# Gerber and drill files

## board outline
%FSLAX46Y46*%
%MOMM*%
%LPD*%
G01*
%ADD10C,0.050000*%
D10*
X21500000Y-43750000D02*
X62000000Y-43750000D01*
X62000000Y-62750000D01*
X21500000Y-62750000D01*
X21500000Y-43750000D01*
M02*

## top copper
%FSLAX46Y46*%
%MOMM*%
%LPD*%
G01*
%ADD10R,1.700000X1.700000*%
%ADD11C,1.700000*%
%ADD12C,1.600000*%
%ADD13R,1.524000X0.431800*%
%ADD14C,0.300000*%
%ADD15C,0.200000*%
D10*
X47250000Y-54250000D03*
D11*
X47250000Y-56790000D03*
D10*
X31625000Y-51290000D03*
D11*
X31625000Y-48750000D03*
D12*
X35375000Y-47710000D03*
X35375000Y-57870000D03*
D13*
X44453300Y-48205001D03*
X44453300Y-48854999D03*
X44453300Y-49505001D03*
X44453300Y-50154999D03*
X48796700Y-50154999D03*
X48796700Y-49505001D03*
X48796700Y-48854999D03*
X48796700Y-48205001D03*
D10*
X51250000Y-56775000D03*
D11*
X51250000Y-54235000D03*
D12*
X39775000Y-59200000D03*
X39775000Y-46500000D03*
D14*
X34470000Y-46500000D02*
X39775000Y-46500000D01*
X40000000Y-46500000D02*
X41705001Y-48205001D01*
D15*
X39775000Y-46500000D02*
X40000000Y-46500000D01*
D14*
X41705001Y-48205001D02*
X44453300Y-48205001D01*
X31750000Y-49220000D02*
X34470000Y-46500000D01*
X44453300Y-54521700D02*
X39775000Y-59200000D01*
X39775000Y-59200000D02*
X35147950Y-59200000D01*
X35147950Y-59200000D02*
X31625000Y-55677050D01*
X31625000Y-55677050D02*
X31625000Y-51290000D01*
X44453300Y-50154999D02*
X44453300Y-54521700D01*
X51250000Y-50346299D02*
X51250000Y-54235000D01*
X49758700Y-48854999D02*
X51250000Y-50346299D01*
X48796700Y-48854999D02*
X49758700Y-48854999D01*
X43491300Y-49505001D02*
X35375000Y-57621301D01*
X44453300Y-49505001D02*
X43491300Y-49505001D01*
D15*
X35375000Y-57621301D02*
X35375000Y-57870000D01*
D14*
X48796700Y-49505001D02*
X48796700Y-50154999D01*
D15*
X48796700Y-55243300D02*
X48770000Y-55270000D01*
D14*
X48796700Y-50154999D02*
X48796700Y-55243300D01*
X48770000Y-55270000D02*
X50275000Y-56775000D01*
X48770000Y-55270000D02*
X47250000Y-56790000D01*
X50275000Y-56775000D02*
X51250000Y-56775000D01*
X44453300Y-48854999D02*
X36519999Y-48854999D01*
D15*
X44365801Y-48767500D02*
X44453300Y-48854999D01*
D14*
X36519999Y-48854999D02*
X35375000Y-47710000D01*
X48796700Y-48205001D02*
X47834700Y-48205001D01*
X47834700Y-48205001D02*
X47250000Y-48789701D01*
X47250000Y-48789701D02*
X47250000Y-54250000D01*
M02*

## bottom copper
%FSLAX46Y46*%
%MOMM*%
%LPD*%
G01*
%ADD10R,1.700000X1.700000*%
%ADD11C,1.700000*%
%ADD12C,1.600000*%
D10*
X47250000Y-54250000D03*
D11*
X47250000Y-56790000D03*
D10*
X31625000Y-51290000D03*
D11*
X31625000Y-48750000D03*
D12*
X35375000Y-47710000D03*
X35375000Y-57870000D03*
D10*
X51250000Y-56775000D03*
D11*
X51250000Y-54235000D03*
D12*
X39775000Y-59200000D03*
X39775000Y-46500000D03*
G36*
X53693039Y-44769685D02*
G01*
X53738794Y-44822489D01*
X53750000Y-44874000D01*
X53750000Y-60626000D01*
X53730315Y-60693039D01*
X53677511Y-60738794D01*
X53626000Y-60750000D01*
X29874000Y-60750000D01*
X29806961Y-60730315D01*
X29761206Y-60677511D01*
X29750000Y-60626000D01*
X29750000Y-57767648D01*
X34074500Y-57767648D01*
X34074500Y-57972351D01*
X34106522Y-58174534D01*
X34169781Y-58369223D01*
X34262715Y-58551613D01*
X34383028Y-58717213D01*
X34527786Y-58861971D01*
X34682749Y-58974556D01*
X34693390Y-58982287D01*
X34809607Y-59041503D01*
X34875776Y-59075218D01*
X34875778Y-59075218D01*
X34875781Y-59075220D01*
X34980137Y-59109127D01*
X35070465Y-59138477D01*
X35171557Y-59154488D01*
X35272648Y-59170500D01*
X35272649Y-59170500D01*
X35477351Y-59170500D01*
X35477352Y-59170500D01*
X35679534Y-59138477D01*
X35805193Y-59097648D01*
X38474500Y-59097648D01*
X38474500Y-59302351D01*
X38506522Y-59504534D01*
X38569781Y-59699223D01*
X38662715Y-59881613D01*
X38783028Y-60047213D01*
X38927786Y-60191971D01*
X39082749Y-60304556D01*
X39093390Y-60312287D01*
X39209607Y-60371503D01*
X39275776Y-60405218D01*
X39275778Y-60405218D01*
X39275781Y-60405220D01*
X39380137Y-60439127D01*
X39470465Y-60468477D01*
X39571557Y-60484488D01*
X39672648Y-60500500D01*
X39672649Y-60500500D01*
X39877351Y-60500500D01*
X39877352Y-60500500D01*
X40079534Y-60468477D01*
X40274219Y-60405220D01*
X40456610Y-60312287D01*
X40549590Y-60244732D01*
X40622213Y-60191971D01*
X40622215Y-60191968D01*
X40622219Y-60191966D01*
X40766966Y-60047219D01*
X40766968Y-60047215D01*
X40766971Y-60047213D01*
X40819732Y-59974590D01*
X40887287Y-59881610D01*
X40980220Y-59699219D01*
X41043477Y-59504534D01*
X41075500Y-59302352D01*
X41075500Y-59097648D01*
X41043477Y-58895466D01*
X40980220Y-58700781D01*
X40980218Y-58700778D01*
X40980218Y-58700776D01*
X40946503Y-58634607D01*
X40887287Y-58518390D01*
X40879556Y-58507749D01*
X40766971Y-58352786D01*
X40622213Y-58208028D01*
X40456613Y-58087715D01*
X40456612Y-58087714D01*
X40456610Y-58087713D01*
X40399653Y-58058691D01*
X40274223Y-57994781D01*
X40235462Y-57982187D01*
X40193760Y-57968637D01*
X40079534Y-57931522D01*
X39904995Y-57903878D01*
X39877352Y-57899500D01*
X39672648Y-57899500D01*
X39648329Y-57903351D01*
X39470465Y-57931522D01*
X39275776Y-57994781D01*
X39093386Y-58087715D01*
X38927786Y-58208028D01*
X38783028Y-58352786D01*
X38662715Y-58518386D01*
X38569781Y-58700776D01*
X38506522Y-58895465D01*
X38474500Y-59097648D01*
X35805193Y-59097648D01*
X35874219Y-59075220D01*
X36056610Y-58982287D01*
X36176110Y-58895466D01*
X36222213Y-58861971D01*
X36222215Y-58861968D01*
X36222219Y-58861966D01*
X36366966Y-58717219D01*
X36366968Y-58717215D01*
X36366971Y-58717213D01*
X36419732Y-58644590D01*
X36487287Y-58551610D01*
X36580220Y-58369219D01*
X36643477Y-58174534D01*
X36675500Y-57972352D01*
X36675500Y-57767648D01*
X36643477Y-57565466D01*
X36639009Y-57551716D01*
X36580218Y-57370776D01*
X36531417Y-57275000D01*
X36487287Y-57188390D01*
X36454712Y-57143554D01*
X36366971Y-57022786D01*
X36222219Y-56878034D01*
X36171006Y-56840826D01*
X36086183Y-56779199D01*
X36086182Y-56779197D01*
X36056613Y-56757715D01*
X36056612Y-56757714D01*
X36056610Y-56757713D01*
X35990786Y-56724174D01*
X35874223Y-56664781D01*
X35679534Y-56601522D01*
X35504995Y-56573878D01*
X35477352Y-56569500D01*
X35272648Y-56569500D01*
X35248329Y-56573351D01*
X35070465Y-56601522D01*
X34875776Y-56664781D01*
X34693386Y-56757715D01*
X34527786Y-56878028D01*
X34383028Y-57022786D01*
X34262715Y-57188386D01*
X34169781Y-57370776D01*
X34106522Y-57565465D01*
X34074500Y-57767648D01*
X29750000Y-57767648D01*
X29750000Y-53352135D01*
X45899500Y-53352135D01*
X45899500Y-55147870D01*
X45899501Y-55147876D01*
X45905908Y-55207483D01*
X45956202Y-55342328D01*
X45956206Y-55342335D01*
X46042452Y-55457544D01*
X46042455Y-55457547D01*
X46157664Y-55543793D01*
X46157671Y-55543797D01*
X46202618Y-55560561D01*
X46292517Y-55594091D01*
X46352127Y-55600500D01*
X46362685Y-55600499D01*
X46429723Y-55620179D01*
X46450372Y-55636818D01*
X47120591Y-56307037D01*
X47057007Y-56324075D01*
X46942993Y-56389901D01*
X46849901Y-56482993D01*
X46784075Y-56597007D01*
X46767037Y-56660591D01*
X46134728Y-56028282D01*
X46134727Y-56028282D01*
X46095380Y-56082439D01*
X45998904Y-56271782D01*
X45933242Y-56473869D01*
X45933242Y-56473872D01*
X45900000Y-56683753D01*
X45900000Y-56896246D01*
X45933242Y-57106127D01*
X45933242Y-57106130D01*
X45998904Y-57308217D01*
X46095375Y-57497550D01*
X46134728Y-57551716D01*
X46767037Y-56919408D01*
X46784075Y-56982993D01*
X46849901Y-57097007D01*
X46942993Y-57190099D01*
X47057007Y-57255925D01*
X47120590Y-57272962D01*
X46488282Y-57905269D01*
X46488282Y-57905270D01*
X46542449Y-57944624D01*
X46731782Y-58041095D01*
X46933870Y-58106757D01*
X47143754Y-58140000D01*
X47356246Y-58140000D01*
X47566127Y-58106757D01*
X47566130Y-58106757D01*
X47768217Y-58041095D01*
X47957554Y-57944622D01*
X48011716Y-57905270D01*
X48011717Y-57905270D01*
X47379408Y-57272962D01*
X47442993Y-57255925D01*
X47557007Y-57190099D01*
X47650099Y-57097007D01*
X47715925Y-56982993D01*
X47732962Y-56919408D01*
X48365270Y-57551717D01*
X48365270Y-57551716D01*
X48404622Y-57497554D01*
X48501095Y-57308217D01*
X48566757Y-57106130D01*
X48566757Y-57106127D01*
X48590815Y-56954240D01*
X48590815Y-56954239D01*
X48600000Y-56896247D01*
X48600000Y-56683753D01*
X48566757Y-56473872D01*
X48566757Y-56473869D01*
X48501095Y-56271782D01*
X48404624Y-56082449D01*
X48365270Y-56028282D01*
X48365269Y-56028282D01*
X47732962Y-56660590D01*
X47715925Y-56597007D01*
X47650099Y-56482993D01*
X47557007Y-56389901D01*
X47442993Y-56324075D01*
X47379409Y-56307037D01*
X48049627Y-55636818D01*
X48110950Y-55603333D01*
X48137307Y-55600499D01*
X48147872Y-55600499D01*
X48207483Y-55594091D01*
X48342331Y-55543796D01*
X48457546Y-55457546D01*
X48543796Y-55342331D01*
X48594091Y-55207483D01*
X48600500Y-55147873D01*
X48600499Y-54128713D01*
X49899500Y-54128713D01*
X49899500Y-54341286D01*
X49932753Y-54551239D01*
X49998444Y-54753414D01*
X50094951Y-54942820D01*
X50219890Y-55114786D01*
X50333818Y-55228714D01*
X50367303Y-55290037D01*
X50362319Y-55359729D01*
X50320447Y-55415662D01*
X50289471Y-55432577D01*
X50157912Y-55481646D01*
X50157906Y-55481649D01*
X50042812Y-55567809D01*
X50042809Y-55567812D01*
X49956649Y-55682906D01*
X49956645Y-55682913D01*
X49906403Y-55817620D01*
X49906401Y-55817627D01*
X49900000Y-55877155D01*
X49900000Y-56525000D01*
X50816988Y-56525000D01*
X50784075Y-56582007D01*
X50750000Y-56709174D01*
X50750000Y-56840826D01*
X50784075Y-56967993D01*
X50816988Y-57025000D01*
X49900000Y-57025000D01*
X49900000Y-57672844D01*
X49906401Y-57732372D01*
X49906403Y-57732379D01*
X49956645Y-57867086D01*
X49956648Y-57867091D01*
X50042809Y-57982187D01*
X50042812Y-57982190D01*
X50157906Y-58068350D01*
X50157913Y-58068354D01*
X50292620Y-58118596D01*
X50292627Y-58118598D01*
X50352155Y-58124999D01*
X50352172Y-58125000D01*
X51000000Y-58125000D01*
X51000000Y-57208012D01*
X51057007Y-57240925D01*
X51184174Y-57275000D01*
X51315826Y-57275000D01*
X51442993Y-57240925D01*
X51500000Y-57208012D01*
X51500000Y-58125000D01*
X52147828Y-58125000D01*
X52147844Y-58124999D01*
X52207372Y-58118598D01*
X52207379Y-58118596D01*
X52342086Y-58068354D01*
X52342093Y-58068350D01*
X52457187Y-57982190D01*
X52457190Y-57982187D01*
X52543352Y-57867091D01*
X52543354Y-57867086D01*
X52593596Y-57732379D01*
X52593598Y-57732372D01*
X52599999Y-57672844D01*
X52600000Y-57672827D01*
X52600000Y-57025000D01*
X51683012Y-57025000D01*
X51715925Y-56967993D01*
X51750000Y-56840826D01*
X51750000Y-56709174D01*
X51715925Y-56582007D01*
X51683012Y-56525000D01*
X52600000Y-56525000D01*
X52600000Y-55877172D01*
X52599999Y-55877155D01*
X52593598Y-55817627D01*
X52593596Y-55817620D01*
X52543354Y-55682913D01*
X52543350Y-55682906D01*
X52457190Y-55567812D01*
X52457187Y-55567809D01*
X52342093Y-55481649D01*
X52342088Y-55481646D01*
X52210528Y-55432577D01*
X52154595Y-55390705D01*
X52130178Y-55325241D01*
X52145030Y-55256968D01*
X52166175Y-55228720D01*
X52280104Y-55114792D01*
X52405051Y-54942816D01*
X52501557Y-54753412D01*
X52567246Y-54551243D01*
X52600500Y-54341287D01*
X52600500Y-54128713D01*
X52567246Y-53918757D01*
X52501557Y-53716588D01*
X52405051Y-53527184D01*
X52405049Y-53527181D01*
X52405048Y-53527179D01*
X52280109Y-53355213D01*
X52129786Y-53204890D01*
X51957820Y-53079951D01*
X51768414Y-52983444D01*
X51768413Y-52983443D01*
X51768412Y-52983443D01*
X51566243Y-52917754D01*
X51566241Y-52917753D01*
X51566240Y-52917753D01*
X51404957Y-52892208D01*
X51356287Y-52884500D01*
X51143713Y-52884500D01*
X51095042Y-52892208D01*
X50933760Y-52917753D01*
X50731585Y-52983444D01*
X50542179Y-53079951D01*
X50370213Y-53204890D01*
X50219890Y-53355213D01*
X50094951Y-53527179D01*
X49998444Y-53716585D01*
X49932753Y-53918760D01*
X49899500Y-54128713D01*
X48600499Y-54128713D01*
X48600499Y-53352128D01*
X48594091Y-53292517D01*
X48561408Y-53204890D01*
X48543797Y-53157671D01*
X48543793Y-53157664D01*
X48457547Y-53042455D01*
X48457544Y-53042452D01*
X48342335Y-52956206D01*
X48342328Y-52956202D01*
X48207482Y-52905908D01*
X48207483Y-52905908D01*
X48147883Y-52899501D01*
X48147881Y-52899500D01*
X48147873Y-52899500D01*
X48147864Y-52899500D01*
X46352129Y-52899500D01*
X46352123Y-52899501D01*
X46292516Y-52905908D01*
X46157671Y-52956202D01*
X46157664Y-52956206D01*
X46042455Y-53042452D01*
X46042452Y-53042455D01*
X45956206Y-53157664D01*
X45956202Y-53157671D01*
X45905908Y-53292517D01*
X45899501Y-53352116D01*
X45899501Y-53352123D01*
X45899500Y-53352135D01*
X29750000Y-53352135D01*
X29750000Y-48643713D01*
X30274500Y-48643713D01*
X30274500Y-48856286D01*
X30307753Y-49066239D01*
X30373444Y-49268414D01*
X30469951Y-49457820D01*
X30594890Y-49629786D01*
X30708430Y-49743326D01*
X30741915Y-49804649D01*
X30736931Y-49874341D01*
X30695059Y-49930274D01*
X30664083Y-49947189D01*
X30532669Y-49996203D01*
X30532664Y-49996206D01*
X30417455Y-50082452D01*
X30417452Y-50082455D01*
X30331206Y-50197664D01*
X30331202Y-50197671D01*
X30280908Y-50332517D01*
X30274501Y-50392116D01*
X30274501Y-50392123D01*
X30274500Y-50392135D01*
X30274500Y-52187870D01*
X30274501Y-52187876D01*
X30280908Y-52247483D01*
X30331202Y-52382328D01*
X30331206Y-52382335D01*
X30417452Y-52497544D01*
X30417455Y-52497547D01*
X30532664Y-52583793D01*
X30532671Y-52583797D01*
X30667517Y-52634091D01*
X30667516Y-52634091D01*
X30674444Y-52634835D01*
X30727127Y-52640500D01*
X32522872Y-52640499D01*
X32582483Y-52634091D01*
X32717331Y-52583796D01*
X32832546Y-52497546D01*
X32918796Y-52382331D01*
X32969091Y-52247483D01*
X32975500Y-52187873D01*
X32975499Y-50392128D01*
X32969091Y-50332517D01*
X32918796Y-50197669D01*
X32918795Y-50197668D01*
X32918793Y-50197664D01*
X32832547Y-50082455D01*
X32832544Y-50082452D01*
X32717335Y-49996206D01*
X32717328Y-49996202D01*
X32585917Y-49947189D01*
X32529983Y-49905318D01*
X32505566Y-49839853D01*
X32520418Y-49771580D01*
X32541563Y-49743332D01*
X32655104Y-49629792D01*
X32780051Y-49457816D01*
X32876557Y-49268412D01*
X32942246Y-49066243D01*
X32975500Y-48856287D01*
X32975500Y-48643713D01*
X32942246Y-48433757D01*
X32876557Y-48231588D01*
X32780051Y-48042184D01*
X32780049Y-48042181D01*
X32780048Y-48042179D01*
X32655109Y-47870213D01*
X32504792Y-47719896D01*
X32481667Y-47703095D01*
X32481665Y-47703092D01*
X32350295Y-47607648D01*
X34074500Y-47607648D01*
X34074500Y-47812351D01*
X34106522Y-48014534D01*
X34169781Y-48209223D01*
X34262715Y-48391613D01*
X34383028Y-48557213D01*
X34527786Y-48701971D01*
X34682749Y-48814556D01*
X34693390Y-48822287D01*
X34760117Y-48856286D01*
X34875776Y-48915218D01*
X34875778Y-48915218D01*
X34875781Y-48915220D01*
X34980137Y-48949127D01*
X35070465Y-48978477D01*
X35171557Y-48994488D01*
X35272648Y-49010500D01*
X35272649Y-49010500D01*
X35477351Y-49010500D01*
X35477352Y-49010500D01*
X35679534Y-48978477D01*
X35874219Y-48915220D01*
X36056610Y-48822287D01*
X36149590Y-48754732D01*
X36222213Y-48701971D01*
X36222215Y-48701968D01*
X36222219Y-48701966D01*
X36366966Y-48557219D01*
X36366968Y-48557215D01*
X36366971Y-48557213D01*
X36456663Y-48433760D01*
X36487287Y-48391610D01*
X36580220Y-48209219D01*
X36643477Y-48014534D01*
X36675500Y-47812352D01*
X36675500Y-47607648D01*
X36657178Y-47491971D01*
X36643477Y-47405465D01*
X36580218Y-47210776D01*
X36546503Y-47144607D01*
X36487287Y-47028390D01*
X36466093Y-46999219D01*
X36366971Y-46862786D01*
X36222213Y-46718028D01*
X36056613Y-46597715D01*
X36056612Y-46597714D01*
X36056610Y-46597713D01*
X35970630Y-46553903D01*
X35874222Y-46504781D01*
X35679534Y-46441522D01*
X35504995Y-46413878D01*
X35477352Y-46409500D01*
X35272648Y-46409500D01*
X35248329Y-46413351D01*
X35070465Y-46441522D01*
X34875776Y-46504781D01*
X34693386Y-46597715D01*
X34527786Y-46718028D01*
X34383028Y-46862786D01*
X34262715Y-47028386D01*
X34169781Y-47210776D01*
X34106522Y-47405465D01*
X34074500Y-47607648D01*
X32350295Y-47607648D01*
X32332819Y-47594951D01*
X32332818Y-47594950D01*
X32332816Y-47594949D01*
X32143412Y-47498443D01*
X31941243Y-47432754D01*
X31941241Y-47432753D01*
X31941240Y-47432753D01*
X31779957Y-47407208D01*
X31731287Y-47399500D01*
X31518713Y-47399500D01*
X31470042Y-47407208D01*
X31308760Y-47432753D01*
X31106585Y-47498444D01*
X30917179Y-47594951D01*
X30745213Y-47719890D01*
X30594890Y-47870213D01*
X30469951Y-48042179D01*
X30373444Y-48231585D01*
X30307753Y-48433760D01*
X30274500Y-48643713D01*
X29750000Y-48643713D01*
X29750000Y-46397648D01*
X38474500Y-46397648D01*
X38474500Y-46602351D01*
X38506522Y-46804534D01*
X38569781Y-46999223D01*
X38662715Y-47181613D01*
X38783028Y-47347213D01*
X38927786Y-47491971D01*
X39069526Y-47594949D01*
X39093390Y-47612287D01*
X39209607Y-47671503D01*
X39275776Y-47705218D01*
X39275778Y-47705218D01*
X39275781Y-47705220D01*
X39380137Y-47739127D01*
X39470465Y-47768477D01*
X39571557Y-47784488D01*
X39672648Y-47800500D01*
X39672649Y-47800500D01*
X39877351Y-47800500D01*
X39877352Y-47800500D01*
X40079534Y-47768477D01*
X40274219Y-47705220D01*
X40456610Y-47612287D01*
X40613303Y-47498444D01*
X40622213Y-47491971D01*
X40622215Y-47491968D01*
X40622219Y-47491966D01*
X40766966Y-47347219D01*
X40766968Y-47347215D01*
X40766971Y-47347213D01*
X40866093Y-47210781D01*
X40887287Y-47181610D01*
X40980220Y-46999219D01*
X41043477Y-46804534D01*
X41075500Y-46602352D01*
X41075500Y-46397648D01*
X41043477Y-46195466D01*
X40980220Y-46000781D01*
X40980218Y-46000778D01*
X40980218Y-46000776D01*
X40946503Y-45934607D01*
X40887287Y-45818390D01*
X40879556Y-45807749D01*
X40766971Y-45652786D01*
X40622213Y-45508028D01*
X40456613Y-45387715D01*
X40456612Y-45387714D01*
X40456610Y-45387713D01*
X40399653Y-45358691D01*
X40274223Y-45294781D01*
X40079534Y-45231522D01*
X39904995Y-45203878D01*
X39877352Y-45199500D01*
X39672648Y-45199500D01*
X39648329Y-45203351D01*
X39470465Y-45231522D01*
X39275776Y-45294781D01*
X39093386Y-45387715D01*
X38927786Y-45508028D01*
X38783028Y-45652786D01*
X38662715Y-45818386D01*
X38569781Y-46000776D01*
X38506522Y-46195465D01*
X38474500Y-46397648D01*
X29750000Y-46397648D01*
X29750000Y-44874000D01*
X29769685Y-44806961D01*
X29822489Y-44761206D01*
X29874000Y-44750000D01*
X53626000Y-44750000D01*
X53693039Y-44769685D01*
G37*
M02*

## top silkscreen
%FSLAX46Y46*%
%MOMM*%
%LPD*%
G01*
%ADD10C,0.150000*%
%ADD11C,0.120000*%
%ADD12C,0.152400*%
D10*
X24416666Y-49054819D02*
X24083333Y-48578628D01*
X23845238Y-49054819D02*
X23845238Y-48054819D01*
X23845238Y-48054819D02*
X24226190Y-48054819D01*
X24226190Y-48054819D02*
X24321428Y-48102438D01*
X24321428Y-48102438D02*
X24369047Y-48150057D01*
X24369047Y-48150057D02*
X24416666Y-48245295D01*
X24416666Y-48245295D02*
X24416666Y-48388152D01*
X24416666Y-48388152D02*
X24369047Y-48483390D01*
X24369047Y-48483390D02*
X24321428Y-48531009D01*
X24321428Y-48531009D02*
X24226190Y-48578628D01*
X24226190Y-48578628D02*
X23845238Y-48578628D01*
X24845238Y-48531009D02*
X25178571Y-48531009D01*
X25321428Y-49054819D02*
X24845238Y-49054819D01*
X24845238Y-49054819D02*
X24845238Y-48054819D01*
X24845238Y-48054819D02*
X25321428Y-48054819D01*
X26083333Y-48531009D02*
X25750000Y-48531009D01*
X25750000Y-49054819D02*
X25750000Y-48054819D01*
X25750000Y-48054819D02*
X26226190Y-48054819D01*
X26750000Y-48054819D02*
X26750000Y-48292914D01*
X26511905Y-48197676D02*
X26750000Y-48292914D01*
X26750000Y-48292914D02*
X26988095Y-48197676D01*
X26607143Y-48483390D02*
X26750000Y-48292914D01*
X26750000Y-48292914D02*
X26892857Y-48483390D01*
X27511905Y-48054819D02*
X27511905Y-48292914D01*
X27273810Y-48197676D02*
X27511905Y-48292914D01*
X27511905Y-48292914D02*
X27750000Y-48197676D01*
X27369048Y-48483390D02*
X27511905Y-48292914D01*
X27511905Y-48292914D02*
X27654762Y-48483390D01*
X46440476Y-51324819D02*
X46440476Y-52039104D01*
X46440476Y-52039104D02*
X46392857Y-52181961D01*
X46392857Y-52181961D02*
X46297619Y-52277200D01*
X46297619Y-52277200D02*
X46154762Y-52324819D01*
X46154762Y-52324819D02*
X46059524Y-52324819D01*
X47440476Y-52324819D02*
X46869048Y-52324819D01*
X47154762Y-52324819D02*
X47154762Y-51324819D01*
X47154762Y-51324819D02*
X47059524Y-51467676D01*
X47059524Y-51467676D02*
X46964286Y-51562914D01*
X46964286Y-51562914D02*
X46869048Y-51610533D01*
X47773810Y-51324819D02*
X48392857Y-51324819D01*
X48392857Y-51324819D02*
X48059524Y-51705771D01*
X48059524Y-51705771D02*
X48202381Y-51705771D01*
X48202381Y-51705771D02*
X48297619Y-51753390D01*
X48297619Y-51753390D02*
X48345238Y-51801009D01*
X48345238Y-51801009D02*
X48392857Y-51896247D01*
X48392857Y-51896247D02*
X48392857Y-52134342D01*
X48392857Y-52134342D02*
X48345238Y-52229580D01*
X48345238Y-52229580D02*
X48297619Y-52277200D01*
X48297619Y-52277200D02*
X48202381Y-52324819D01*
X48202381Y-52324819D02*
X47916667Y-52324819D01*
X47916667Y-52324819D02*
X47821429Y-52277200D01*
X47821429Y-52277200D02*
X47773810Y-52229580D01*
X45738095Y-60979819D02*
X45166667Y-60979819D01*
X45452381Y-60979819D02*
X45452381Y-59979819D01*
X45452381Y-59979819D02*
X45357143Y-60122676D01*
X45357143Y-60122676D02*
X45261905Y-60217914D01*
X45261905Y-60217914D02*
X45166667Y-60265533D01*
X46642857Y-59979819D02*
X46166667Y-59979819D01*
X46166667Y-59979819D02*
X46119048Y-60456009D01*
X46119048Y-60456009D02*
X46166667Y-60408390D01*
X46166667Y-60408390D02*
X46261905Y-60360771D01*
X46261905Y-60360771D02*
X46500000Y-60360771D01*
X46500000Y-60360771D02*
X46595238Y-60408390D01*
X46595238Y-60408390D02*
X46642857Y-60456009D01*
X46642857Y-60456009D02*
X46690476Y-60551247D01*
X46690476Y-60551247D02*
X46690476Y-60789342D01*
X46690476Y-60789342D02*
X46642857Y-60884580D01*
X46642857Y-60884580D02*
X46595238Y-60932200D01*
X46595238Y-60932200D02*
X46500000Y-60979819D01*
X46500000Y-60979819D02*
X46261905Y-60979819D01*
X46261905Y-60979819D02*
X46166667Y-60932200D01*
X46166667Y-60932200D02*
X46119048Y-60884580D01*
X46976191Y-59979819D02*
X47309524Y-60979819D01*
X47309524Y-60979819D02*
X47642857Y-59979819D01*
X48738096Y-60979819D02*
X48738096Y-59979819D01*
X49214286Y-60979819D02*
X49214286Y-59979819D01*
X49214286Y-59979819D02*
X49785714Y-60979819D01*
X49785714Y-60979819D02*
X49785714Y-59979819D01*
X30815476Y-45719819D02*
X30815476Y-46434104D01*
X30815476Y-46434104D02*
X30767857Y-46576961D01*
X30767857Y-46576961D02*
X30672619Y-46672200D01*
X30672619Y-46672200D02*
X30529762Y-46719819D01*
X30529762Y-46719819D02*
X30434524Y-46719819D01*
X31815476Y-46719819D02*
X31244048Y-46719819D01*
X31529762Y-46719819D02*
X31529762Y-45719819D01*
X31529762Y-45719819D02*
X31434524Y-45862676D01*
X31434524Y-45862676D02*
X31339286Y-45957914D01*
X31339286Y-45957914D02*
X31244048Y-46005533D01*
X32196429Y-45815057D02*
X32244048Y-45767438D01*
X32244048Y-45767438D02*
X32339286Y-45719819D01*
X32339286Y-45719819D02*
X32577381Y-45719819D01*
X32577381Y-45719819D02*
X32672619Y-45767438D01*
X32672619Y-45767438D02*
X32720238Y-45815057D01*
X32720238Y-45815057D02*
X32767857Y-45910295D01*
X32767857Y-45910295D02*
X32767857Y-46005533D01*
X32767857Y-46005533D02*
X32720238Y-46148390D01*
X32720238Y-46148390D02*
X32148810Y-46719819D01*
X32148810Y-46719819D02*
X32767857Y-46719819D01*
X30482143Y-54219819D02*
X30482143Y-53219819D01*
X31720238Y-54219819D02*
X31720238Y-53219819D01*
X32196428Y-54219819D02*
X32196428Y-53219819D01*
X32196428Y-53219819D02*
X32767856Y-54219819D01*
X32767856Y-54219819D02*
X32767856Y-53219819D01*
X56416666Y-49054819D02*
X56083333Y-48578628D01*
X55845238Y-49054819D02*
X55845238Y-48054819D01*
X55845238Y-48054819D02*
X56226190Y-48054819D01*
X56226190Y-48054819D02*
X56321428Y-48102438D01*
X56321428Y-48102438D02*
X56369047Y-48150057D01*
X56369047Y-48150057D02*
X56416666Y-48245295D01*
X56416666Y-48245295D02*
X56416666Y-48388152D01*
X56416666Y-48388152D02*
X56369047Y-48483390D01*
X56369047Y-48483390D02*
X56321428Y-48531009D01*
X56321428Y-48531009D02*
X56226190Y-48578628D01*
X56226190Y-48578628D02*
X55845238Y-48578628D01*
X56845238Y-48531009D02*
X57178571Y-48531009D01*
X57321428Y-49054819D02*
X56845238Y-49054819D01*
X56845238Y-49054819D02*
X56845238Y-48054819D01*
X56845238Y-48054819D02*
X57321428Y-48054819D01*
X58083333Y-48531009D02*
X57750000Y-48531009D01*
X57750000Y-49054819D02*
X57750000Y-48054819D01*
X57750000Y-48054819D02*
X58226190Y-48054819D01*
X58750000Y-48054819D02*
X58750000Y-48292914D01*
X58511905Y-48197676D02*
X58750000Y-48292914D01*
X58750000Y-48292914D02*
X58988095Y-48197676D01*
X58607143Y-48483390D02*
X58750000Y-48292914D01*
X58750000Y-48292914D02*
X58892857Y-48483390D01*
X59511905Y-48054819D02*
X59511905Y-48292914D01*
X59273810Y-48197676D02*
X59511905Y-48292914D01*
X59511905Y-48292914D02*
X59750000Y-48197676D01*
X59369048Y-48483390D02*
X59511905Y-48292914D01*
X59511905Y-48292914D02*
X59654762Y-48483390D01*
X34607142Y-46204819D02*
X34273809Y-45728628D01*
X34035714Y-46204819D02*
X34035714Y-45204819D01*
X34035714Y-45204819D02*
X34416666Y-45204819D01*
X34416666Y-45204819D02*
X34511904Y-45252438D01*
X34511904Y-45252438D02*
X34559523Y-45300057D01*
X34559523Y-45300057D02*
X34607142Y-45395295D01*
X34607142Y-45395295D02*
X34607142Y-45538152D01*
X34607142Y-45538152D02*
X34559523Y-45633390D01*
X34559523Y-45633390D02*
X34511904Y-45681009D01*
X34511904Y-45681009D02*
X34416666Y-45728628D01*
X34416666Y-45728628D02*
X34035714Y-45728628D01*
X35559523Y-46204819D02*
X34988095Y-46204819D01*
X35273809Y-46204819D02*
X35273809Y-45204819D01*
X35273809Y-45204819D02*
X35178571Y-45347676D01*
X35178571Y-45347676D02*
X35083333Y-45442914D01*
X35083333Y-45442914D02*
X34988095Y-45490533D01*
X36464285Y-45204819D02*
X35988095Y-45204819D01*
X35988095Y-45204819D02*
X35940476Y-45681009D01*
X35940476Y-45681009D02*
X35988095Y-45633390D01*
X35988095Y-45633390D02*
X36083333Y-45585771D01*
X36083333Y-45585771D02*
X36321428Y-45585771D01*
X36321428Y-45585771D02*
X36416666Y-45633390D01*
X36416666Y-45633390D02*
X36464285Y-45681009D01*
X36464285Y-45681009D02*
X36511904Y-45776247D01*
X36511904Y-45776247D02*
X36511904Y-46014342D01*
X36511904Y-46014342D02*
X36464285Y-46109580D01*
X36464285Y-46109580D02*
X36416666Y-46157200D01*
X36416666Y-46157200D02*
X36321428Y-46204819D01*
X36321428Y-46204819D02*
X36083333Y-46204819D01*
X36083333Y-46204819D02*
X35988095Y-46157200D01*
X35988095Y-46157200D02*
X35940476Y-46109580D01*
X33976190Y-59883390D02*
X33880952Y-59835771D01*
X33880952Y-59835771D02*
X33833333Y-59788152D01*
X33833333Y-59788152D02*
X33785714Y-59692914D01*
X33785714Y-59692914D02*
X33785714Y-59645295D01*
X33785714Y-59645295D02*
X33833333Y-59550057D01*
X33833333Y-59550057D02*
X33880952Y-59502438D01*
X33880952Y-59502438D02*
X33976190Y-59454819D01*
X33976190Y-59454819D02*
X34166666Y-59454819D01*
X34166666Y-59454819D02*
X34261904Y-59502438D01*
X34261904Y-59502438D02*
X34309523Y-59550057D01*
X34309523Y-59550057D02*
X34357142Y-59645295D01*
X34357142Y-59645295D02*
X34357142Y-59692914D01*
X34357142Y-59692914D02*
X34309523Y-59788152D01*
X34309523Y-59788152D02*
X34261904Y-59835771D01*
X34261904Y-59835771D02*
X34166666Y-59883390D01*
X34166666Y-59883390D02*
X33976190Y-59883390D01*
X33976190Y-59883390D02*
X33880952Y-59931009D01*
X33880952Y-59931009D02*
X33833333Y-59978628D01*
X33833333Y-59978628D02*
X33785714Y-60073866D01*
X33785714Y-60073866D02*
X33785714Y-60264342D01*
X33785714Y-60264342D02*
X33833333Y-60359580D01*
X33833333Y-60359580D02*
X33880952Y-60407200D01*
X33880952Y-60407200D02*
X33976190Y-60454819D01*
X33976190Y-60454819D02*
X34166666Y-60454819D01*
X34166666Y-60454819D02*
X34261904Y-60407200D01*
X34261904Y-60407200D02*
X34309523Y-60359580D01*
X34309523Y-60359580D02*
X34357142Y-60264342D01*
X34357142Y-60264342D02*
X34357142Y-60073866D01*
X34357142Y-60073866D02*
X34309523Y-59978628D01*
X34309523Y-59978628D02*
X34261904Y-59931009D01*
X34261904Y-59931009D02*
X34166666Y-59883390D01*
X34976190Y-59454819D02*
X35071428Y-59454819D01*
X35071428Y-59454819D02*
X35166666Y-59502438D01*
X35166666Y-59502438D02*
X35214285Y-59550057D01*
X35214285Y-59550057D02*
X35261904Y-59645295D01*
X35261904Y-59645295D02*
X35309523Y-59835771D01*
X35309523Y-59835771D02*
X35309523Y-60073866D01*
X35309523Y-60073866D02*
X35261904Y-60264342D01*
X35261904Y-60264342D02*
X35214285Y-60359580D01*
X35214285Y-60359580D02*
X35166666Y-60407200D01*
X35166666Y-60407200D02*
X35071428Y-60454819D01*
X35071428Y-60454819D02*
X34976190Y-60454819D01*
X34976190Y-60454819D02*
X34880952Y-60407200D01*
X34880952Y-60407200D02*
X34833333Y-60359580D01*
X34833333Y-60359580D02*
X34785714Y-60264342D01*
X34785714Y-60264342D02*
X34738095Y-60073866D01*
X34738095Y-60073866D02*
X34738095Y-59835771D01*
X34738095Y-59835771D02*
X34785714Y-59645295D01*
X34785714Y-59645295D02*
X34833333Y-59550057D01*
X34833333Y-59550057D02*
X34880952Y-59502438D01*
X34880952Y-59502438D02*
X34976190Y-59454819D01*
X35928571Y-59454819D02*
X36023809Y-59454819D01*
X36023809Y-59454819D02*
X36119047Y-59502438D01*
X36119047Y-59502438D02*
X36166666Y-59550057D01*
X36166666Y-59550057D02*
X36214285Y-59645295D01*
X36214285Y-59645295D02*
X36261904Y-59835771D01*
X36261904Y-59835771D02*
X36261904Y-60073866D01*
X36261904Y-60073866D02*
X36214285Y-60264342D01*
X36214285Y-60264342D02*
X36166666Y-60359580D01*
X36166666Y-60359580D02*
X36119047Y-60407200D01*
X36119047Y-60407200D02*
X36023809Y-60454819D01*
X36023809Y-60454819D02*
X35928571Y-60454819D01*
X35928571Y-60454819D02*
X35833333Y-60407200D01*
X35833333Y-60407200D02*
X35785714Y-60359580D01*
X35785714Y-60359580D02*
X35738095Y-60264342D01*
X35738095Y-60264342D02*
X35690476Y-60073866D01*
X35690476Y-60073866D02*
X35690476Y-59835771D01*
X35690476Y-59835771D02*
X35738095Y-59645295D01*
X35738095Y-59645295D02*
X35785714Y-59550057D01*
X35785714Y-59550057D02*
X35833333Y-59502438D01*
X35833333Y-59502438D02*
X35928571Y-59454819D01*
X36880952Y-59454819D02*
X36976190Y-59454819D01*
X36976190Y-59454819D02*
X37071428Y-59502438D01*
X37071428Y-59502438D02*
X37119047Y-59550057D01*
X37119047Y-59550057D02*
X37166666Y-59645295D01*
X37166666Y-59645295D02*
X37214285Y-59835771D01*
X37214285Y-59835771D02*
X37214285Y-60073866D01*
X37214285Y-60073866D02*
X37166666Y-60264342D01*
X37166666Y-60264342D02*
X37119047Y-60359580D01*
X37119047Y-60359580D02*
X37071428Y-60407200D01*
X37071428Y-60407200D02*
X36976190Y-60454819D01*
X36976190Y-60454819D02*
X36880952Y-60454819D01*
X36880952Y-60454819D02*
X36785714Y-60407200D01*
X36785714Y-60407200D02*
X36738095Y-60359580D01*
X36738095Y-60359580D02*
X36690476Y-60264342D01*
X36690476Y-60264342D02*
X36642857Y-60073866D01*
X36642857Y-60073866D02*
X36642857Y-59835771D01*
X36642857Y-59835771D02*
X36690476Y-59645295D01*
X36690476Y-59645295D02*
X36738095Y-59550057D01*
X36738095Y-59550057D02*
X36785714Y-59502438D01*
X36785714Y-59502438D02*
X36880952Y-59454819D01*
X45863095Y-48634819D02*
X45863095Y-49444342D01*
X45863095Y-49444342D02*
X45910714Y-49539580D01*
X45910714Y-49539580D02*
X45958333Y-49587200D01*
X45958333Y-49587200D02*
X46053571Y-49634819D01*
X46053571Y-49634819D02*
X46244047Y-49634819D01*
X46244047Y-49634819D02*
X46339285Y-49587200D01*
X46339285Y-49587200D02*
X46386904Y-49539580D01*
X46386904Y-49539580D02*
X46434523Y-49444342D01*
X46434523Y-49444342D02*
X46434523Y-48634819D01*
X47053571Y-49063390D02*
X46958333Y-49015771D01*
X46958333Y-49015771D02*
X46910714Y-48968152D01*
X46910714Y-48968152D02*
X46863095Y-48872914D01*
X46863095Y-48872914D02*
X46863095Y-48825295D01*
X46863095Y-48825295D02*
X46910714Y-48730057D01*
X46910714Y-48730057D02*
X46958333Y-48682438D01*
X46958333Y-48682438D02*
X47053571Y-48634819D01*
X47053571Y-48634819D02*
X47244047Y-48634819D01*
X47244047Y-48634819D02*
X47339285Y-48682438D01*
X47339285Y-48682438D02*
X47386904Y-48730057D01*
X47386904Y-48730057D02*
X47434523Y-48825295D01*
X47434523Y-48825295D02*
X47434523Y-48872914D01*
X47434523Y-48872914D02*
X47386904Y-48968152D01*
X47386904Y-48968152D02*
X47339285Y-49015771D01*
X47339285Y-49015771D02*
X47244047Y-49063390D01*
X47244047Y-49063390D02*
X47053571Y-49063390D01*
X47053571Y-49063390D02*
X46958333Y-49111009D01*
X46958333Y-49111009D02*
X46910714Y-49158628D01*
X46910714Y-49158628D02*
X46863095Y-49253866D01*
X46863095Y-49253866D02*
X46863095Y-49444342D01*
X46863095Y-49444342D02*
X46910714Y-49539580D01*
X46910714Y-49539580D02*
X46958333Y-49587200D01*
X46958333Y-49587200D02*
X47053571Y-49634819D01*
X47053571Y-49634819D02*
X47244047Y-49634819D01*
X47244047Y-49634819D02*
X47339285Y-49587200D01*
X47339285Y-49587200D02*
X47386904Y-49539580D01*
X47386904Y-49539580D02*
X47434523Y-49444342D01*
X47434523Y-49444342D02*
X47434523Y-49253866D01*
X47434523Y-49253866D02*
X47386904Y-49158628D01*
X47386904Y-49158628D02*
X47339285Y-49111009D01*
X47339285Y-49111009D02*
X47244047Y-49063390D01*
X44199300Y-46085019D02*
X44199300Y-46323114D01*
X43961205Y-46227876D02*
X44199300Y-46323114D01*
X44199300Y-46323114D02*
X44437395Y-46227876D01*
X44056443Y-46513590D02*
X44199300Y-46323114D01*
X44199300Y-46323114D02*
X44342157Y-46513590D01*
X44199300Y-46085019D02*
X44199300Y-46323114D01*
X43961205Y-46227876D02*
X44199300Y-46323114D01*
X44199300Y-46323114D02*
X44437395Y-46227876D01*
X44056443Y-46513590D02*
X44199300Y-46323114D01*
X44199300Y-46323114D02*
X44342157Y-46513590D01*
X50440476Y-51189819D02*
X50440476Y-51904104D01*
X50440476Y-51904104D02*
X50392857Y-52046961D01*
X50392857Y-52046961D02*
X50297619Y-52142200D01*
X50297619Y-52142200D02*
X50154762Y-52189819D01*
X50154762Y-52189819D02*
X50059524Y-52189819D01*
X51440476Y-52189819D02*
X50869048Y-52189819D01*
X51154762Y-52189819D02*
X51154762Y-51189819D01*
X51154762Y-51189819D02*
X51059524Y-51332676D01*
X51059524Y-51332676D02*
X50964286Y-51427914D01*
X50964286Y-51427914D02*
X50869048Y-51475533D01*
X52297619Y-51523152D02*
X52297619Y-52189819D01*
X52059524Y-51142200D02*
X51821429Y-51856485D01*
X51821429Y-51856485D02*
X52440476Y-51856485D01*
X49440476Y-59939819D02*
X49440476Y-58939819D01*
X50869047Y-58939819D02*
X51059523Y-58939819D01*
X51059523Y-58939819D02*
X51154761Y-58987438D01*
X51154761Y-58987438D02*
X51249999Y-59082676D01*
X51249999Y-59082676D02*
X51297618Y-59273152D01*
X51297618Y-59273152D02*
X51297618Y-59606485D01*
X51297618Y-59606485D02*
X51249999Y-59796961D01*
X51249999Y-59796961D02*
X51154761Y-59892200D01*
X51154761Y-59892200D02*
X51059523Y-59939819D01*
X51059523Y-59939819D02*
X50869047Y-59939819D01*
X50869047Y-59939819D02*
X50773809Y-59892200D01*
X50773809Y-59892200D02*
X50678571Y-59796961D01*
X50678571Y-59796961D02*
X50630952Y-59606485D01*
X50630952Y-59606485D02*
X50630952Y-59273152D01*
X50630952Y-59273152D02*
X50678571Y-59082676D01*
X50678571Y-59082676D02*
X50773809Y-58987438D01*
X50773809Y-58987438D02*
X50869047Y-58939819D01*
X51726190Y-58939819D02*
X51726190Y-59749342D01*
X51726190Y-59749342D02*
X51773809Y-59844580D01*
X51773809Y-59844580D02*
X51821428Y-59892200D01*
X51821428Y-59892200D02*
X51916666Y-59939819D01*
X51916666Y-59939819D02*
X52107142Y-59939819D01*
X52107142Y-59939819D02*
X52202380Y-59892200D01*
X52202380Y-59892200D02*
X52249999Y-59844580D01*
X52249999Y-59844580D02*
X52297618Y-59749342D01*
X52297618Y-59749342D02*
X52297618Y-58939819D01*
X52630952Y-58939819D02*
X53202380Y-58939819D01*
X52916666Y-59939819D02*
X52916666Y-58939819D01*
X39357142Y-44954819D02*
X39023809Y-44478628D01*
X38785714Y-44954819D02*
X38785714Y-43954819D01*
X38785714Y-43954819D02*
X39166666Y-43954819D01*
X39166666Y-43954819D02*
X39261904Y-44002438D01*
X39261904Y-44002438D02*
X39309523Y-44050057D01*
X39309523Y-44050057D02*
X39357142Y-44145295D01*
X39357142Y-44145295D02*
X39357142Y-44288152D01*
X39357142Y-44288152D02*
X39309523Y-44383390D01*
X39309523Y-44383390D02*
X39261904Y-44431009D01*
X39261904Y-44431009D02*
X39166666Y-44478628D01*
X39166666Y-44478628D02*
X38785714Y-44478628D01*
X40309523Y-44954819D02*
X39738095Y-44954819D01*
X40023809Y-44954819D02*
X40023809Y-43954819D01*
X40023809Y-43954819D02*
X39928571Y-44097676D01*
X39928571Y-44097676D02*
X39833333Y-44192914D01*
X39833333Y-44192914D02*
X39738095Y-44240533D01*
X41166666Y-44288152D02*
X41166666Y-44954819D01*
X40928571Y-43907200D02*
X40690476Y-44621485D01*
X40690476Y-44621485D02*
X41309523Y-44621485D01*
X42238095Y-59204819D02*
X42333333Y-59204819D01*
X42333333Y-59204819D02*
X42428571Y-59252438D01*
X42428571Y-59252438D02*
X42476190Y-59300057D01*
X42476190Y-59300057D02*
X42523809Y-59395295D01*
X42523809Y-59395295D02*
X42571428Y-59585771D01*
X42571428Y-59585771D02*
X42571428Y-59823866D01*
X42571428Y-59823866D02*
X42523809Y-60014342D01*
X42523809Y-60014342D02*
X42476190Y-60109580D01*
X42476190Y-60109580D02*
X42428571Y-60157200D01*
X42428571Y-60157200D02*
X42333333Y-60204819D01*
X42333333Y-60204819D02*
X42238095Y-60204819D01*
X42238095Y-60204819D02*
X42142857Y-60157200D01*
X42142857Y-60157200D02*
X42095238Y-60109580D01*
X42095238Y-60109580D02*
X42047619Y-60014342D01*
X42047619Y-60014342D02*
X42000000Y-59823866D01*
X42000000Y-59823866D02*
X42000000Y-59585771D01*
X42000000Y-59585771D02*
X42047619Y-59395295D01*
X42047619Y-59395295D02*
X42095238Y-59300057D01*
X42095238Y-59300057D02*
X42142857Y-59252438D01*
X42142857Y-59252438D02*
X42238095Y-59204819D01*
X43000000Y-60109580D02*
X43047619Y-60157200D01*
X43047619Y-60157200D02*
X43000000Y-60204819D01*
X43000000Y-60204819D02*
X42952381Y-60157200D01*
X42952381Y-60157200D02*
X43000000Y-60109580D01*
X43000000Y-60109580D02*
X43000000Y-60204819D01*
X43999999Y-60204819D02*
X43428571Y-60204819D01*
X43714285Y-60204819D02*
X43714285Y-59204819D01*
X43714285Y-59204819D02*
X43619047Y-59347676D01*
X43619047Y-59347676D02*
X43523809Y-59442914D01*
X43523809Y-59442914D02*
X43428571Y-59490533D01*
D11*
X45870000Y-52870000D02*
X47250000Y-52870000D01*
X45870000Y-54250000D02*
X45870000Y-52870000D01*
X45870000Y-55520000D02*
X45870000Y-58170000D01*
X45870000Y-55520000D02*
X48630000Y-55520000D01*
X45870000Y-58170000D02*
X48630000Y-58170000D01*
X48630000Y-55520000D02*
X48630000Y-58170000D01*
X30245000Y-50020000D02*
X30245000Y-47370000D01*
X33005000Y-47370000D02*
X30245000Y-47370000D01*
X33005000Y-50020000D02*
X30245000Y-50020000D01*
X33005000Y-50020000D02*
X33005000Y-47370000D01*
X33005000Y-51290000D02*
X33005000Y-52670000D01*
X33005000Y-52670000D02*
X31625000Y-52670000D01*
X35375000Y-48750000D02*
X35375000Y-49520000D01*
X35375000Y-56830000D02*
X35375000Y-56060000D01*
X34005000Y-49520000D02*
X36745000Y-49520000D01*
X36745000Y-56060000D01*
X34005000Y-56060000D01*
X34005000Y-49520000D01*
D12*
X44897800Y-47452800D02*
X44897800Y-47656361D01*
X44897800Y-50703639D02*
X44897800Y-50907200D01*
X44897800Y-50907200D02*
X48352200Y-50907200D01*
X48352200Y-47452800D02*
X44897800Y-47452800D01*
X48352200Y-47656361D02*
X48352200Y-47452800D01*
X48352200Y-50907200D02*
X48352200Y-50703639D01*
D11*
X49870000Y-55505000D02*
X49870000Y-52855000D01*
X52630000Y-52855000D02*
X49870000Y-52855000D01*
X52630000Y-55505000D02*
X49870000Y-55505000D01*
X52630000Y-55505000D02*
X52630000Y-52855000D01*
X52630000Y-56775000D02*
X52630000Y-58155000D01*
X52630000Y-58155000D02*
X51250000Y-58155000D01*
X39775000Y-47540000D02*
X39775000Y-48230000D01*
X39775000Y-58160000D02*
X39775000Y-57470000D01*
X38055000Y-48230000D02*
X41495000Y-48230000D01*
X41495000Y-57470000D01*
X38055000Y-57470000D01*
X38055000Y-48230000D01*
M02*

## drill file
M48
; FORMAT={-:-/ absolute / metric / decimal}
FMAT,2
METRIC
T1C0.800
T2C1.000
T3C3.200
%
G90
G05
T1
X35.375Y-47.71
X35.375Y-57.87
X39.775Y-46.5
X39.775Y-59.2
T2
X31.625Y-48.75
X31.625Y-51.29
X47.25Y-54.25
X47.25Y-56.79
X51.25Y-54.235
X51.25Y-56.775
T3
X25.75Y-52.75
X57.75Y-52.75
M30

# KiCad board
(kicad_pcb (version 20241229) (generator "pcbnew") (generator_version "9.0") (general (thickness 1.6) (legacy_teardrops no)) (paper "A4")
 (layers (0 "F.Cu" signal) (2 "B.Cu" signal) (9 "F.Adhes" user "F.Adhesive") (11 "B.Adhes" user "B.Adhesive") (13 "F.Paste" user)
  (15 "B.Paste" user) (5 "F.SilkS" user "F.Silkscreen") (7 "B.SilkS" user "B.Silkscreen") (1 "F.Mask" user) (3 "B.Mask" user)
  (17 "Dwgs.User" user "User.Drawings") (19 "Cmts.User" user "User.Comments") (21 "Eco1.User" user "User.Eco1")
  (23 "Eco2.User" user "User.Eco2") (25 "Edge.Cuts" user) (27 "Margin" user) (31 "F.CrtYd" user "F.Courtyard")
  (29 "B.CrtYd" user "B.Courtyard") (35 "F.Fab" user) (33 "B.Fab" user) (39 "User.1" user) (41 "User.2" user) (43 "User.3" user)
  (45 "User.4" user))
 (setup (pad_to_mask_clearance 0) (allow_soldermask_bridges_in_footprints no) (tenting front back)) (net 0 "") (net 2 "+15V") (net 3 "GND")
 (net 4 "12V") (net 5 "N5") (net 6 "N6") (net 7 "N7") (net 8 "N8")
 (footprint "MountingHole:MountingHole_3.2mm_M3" (layer "F.Cu") (at 25.75 52.75)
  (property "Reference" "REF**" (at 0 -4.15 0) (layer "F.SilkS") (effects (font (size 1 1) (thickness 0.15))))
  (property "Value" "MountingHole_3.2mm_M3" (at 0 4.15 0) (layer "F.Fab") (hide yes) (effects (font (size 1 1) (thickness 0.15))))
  (pad "" np_thru_hole circle (at 0 0) (size 3.2 3.2) (drill 3.2) (layers "*.Cu" "*.Mask")))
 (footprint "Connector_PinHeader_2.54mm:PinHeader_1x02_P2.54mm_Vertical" (layer "F.Cu") (at 47.25 54.25)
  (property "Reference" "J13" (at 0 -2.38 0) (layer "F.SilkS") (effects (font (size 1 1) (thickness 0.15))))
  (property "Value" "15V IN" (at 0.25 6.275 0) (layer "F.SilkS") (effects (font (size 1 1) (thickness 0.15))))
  (fp_line (start -1.38 -1.38) (end 0 -1.38) (stroke (width 0.12) (type solid)) (layer "F.SilkS") (net 1))
  (fp_line (start -1.38 0) (end -1.38 -1.38) (stroke (width 0.12) (type solid)) (layer "F.SilkS") (net 1))
  (fp_line (start -1.38 1.27) (end -1.38 3.92) (stroke (width 0.12) (type solid)) (layer "F.SilkS") (net 1))
  (fp_line (start -1.38 1.27) (end 1.38 1.27) (stroke (width 0.12) (type solid)) (layer "F.SilkS") (net 1))
  (fp_line (start -1.38 3.92) (end 1.38 3.92) (stroke (width 0.12) (type solid)) (layer "F.SilkS") (net 1))
  (fp_line (start 1.38 1.27) (end 1.38 3.92) (stroke (width 0.12) (type solid)) (layer "F.SilkS") (net 1))
  (pad "1" thru_hole rect (at 0 0) (size 1.7 1.7) (drill 1) (layers "*.Cu" "*.Mask") (remove_unused_layers no) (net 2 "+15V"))
  (pad "2" thru_hole circle (at 0 2.54) (size 1.7 1.7) (drill 1) (layers "*.Cu" "*.Mask") (remove_unused_layers no) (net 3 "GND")))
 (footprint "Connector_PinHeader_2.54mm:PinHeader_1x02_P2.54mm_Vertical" (layer "F.Cu") (at 31.625 51.29 180)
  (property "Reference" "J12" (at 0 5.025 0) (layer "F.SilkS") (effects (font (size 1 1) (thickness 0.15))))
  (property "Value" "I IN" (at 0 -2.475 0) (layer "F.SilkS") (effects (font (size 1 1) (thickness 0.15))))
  (fp_line (start 1.38 1.27) (end 1.38 3.92) (stroke (width 0.12) (type solid)) (layer "F.SilkS") (net 1))
  (fp_line (start -1.38 3.92) (end 1.38 3.92) (stroke (width 0.12) (type solid)) (layer "F.SilkS") (net 1))
  (fp_line (start -1.38 1.27) (end 1.38 1.27) (stroke (width 0.12) (type solid)) (layer "F.SilkS") (net 1))
  (fp_line (start -1.38 1.27) (end -1.38 3.92) (stroke (width 0.12) (type solid)) (layer "F.SilkS") (net 1))
  (fp_line (start -1.38 0) (end -1.38 -1.38) (stroke (width 0.12) (type solid)) (layer "F.SilkS") (net 1))
  (fp_line (start -1.38 -1.38) (end 0 -1.38) (stroke (width 0.12) (type solid)) (layer "F.SilkS") (net 1))
  (pad "1" thru_hole rect (at 0 0 180) (size 1.7 1.7) (drill 1) (layers "*.Cu" "*.Mask") (remove_unused_layers no) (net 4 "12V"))
  (pad "2" thru_hole circle (at 0 2.54 180) (size 1.7 1.7) (drill 1) (layers "*.Cu" "*.Mask") (remove_unused_layers no) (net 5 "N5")))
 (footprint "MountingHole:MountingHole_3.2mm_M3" (layer "F.Cu") (at 57.75 52.75)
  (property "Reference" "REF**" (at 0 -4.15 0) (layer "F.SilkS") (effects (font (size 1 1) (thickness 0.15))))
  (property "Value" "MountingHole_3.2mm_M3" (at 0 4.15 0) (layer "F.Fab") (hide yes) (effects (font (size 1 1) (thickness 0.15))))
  (pad "" np_thru_hole circle (at 0 0) (size 3.2 3.2) (drill 3.2) (layers "*.Cu" "*.Mask")))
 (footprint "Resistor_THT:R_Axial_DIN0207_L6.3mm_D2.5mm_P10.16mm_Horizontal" (layer "F.Cu") (at 35.375 47.71 -90)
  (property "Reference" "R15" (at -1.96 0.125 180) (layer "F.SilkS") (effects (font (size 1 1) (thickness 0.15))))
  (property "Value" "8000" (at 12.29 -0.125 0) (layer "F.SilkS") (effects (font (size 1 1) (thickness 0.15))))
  (fp_line (start 1.04 0) (end 1.81 0) (stroke (width 0.12) (type solid)) (layer "F.SilkS"))
  (fp_line (start 9.12 0) (end 8.35 0) (stroke (width 0.12) (type solid)) (layer "F.SilkS"))
  (fp_rect (start 1.81 -1.37) (end 8.35 1.37) (stroke (width 0.12) (type solid)) (fill no) (layer "F.SilkS"))
  (pad "1" thru_hole circle (at 0 0 270) (size 1.6 1.6) (drill 0.8) (layers "*.Cu" "*.Mask") (remove_unused_layers no) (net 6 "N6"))
  (pad "2" thru_hole circle (at 10.16 0 270) (size 1.6 1.6) (drill 0.8) (layers "*.Cu" "*.Mask") (remove_unused_layers no) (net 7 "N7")))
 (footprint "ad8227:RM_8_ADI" (layer "F.Cu") (at 46.625 49.18)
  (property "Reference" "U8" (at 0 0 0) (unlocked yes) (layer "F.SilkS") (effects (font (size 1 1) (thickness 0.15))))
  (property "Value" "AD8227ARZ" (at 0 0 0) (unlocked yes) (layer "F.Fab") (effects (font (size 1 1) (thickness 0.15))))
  (fp_line (start -1.7272 -1.7272) (end -1.7272 -1.523639) (stroke (width 0.1524) (type solid)) (layer "F.SilkS") (net 1))
  (fp_line (start -1.7272 1.523639) (end -1.7272 1.7272) (stroke (width 0.1524) (type solid)) (layer "F.SilkS") (net 1))
  (fp_line (start -1.7272 1.7272) (end 1.7272 1.7272) (stroke (width 0.1524) (type solid)) (layer "F.SilkS") (net 1))
  (fp_line (start 1.7272 -1.7272) (end -1.7272 -1.7272) (stroke (width 0.1524) (type solid)) (layer "F.SilkS") (net 1))
  (fp_line (start 1.7272 -1.523639) (end 1.7272 -1.7272) (stroke (width 0.1524) (type solid)) (layer "F.SilkS") (net 1))
  (fp_line (start 1.7272 1.7272) (end 1.7272 1.523639) (stroke (width 0.1524) (type solid)) (layer "F.SilkS") (net 1))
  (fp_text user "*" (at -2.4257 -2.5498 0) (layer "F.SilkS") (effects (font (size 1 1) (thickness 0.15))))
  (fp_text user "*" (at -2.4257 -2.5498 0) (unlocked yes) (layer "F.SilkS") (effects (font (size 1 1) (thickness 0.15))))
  (pad "1" smd rect (at -2.1717 -0.974999) (size 1.524 0.4318) (layers "F.Cu" "F.Mask" "F.Paste") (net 5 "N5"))
  (pad "2" smd rect (at -2.1717 -0.325001) (size 1.524 0.4318) (layers "F.Cu" "F.Mask" "F.Paste") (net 6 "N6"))
  (pad "3" smd rect (at -2.1717 0.325001) (size 1.524 0.4318) (layers "F.Cu" "F.Mask" "F.Paste") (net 7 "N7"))
  (pad "4" smd rect (at -2.1717 0.974999) (size 1.524 0.4318) (layers "F.Cu" "F.Mask" "F.Paste") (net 4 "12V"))
  (pad "5" smd rect (at 2.1717 0.974999) (size 1.524 0.4318) (layers "F.Cu" "F.Mask" "F.Paste") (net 3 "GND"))
  (pad "6" smd rect (at 2.1717 0.325001) (size 1.524 0.4318) (layers "F.Cu" "F.Mask" "F.Paste") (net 3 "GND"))
  (pad "7" smd rect (at 2.1717 -0.325001) (size 1.524 0.4318) (layers "F.Cu" "F.Mask" "F.Paste") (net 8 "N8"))
  (pad "8" smd rect (at 2.1717 -0.974999) (size 1.524 0.4318) (layers "F.Cu" "F.Mask" "F.Paste") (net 2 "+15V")))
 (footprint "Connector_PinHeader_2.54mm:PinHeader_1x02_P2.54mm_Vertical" (layer "F.Cu") (at 51.25 56.775 180)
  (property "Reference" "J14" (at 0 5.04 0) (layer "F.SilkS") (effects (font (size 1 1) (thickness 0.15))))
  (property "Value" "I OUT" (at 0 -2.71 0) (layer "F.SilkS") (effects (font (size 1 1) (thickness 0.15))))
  (fp_line (start 1.38 1.27) (end 1.38 3.92) (stroke (width 0.12) (type solid)) (layer "F.SilkS") (net 1))
  (fp_line (start -1.38 3.92) (end 1.38 3.92) (stroke (width 0.12) (type solid)) (layer "F.SilkS") (net 1))
  (fp_line (start -1.38 1.27) (end 1.38 1.27) (stroke (width 0.12) (type solid)) (layer "F.SilkS") (net 1))
  (fp_line (start -1.38 1.27) (end -1.38 3.92) (stroke (width 0.12) (type solid)) (layer "F.SilkS") (net 1))
  (fp_line (start -1.38 0) (end -1.38 -1.38) (stroke (width 0.12) (type solid)) (layer "F.SilkS") (net 1))
  (fp_line (start -1.38 -1.38) (end 0 -1.38) (stroke (width 0.12) (type solid)) (layer "F.SilkS") (net 1))
  (pad "1" thru_hole rect (at 0 0 180) (size 1.7 1.7) (drill 1) (layers "*.Cu" "*.Mask") (remove_unused_layers no) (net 3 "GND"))
  (pad "2" thru_hole circle (at 0 2.54 180) (size 1.7 1.7) (drill 1) (layers "*.Cu" "*.Mask") (remove_unused_layers no) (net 8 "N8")))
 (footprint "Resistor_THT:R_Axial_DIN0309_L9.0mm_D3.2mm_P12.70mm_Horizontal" (layer "F.Cu") (at 39.775 59.2 90)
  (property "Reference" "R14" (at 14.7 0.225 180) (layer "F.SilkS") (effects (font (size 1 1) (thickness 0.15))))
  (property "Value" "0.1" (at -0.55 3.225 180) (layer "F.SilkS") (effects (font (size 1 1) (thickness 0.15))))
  (fp_line (start 11.66 0) (end 10.97 0) (stroke (width 0.12) (type solid)) (layer "F.SilkS"))
  (fp_line (start 1.04 0) (end 1.73 0) (stroke (width 0.12) (type solid)) (layer "F.SilkS"))
  (fp_rect (start 1.73 -1.72) (end 10.97 1.72) (stroke (width 0.12) (type solid)) (fill no) (layer "F.SilkS"))
  (pad "1" thru_hole circle (at 0 0 90) (size 1.6 1.6) (drill 0.8) (layers "*.Cu" "*.Mask") (remove_unused_layers no) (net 4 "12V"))
  (pad "2" thru_hole circle (at 12.7 0 90) (size 1.6 1.6) (drill 0.8) (layers "*.Cu" "*.Mask") (remove_unused_layers no) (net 5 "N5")))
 (gr_rect (start 21.5 43.75) (end 62 62.75) (stroke (width 0.05) (type default)) (fill no) (layer "Edge.Cuts"))
 (segment (start 34.47 46.5) (end 39.775 46.5) (width 0.3) (layer "F.Cu") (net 5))
 (segment (start 40 46.5) (end 41.705001 48.205001) (width 0.3) (layer "F.Cu") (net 5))
 (segment (start 39.775 46.5) (end 40 46.5) (width 0.2) (layer "F.Cu") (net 5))
 (segment (start 41.705001 48.205001) (end 44.4533 48.205001) (width 0.3) (layer "F.Cu") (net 5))
 (segment (start 31.75 49.22) (end 34.47 46.5) (width 0.3) (layer "F.Cu") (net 5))
 (segment (start 44.4533 54.5217) (end 39.775 59.2) (width 0.3) (layer "F.Cu") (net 4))
 (segment (start 39.775 59.2) (end 35.14795 59.2) (width 0.3) (layer "F.Cu") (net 4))
 (segment (start 35.14795 59.2) (end 31.625 55.67705) (width 0.3) (layer "F.Cu") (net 4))
 (segment (start 31.625 55.67705) (end 31.625 51.29) (width 0.3) (layer "F.Cu") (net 4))
 (segment (start 44.4533 50.154999) (end 44.4533 54.5217) (width 0.3) (layer "F.Cu") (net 4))
 (segment (start 51.25 50.346299) (end 51.25 54.235) (width 0.3) (layer "F.Cu") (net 8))
 (segment (start 49.7587 48.854999) (end 51.25 50.346299) (width 0.3) (layer "F.Cu") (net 8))
 (segment (start 48.7967 48.854999) (end 49.7587 48.854999) (width 0.3) (layer "F.Cu") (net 8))
 (segment (start 43.4913 49.505001) (end 35.375 57.621301) (width 0.3) (layer "F.Cu") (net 7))
 (segment (start 44.4533 49.505001) (end 43.4913 49.505001) (width 0.3) (layer "F.Cu") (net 7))
 (segment (start 35.375 57.621301) (end 35.375 57.87) (width 0.2) (layer "F.Cu") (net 7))
 (segment (start 48.7967 49.505001) (end 48.7967 50.154999) (width 0.3) (layer "F.Cu") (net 3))
 (segment (start 48.7967 55.2433) (end 48.77 55.27) (width 0.2) (layer "F.Cu") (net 3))
 (segment (start 48.7967 50.154999) (end 48.7967 55.2433) (width 0.3) (layer "F.Cu") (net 3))
 (segment (start 48.77 55.27) (end 50.275 56.775) (width 0.3) (layer "F.Cu") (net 3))
 (segment (start 48.77 55.27) (end 47.25 56.79) (width 0.3) (layer "F.Cu") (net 3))
 (segment (start 50.275 56.775) (end 51.25 56.775) (width 0.3) (layer "F.Cu") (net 3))
 (segment (start 44.4533 48.854999) (end 36.519999 48.854999) (width 0.3) (layer "F.Cu") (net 6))
 (segment (start 44.365801 48.7675) (end 44.4533 48.854999) (width 0.2) (layer "F.Cu") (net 6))
 (segment (start 36.519999 48.854999) (end 35.375 47.71) (width 0.3) (layer "F.Cu") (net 6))
 (segment (start 48.7967 48.205001) (end 47.8347 48.205001) (width 0.3) (layer "F.Cu") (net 2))
 (segment (start 47.8347 48.205001) (end 47.25 48.789701) (width 0.3) (layer "F.Cu") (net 2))
 (segment (start 47.25 48.789701) (end 47.25 54.25) (width 0.3) (layer "F.Cu") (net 2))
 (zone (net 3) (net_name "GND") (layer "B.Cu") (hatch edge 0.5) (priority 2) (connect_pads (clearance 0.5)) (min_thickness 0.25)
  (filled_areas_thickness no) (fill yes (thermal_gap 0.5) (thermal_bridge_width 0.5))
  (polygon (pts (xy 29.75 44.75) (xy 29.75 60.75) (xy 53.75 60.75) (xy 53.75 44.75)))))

